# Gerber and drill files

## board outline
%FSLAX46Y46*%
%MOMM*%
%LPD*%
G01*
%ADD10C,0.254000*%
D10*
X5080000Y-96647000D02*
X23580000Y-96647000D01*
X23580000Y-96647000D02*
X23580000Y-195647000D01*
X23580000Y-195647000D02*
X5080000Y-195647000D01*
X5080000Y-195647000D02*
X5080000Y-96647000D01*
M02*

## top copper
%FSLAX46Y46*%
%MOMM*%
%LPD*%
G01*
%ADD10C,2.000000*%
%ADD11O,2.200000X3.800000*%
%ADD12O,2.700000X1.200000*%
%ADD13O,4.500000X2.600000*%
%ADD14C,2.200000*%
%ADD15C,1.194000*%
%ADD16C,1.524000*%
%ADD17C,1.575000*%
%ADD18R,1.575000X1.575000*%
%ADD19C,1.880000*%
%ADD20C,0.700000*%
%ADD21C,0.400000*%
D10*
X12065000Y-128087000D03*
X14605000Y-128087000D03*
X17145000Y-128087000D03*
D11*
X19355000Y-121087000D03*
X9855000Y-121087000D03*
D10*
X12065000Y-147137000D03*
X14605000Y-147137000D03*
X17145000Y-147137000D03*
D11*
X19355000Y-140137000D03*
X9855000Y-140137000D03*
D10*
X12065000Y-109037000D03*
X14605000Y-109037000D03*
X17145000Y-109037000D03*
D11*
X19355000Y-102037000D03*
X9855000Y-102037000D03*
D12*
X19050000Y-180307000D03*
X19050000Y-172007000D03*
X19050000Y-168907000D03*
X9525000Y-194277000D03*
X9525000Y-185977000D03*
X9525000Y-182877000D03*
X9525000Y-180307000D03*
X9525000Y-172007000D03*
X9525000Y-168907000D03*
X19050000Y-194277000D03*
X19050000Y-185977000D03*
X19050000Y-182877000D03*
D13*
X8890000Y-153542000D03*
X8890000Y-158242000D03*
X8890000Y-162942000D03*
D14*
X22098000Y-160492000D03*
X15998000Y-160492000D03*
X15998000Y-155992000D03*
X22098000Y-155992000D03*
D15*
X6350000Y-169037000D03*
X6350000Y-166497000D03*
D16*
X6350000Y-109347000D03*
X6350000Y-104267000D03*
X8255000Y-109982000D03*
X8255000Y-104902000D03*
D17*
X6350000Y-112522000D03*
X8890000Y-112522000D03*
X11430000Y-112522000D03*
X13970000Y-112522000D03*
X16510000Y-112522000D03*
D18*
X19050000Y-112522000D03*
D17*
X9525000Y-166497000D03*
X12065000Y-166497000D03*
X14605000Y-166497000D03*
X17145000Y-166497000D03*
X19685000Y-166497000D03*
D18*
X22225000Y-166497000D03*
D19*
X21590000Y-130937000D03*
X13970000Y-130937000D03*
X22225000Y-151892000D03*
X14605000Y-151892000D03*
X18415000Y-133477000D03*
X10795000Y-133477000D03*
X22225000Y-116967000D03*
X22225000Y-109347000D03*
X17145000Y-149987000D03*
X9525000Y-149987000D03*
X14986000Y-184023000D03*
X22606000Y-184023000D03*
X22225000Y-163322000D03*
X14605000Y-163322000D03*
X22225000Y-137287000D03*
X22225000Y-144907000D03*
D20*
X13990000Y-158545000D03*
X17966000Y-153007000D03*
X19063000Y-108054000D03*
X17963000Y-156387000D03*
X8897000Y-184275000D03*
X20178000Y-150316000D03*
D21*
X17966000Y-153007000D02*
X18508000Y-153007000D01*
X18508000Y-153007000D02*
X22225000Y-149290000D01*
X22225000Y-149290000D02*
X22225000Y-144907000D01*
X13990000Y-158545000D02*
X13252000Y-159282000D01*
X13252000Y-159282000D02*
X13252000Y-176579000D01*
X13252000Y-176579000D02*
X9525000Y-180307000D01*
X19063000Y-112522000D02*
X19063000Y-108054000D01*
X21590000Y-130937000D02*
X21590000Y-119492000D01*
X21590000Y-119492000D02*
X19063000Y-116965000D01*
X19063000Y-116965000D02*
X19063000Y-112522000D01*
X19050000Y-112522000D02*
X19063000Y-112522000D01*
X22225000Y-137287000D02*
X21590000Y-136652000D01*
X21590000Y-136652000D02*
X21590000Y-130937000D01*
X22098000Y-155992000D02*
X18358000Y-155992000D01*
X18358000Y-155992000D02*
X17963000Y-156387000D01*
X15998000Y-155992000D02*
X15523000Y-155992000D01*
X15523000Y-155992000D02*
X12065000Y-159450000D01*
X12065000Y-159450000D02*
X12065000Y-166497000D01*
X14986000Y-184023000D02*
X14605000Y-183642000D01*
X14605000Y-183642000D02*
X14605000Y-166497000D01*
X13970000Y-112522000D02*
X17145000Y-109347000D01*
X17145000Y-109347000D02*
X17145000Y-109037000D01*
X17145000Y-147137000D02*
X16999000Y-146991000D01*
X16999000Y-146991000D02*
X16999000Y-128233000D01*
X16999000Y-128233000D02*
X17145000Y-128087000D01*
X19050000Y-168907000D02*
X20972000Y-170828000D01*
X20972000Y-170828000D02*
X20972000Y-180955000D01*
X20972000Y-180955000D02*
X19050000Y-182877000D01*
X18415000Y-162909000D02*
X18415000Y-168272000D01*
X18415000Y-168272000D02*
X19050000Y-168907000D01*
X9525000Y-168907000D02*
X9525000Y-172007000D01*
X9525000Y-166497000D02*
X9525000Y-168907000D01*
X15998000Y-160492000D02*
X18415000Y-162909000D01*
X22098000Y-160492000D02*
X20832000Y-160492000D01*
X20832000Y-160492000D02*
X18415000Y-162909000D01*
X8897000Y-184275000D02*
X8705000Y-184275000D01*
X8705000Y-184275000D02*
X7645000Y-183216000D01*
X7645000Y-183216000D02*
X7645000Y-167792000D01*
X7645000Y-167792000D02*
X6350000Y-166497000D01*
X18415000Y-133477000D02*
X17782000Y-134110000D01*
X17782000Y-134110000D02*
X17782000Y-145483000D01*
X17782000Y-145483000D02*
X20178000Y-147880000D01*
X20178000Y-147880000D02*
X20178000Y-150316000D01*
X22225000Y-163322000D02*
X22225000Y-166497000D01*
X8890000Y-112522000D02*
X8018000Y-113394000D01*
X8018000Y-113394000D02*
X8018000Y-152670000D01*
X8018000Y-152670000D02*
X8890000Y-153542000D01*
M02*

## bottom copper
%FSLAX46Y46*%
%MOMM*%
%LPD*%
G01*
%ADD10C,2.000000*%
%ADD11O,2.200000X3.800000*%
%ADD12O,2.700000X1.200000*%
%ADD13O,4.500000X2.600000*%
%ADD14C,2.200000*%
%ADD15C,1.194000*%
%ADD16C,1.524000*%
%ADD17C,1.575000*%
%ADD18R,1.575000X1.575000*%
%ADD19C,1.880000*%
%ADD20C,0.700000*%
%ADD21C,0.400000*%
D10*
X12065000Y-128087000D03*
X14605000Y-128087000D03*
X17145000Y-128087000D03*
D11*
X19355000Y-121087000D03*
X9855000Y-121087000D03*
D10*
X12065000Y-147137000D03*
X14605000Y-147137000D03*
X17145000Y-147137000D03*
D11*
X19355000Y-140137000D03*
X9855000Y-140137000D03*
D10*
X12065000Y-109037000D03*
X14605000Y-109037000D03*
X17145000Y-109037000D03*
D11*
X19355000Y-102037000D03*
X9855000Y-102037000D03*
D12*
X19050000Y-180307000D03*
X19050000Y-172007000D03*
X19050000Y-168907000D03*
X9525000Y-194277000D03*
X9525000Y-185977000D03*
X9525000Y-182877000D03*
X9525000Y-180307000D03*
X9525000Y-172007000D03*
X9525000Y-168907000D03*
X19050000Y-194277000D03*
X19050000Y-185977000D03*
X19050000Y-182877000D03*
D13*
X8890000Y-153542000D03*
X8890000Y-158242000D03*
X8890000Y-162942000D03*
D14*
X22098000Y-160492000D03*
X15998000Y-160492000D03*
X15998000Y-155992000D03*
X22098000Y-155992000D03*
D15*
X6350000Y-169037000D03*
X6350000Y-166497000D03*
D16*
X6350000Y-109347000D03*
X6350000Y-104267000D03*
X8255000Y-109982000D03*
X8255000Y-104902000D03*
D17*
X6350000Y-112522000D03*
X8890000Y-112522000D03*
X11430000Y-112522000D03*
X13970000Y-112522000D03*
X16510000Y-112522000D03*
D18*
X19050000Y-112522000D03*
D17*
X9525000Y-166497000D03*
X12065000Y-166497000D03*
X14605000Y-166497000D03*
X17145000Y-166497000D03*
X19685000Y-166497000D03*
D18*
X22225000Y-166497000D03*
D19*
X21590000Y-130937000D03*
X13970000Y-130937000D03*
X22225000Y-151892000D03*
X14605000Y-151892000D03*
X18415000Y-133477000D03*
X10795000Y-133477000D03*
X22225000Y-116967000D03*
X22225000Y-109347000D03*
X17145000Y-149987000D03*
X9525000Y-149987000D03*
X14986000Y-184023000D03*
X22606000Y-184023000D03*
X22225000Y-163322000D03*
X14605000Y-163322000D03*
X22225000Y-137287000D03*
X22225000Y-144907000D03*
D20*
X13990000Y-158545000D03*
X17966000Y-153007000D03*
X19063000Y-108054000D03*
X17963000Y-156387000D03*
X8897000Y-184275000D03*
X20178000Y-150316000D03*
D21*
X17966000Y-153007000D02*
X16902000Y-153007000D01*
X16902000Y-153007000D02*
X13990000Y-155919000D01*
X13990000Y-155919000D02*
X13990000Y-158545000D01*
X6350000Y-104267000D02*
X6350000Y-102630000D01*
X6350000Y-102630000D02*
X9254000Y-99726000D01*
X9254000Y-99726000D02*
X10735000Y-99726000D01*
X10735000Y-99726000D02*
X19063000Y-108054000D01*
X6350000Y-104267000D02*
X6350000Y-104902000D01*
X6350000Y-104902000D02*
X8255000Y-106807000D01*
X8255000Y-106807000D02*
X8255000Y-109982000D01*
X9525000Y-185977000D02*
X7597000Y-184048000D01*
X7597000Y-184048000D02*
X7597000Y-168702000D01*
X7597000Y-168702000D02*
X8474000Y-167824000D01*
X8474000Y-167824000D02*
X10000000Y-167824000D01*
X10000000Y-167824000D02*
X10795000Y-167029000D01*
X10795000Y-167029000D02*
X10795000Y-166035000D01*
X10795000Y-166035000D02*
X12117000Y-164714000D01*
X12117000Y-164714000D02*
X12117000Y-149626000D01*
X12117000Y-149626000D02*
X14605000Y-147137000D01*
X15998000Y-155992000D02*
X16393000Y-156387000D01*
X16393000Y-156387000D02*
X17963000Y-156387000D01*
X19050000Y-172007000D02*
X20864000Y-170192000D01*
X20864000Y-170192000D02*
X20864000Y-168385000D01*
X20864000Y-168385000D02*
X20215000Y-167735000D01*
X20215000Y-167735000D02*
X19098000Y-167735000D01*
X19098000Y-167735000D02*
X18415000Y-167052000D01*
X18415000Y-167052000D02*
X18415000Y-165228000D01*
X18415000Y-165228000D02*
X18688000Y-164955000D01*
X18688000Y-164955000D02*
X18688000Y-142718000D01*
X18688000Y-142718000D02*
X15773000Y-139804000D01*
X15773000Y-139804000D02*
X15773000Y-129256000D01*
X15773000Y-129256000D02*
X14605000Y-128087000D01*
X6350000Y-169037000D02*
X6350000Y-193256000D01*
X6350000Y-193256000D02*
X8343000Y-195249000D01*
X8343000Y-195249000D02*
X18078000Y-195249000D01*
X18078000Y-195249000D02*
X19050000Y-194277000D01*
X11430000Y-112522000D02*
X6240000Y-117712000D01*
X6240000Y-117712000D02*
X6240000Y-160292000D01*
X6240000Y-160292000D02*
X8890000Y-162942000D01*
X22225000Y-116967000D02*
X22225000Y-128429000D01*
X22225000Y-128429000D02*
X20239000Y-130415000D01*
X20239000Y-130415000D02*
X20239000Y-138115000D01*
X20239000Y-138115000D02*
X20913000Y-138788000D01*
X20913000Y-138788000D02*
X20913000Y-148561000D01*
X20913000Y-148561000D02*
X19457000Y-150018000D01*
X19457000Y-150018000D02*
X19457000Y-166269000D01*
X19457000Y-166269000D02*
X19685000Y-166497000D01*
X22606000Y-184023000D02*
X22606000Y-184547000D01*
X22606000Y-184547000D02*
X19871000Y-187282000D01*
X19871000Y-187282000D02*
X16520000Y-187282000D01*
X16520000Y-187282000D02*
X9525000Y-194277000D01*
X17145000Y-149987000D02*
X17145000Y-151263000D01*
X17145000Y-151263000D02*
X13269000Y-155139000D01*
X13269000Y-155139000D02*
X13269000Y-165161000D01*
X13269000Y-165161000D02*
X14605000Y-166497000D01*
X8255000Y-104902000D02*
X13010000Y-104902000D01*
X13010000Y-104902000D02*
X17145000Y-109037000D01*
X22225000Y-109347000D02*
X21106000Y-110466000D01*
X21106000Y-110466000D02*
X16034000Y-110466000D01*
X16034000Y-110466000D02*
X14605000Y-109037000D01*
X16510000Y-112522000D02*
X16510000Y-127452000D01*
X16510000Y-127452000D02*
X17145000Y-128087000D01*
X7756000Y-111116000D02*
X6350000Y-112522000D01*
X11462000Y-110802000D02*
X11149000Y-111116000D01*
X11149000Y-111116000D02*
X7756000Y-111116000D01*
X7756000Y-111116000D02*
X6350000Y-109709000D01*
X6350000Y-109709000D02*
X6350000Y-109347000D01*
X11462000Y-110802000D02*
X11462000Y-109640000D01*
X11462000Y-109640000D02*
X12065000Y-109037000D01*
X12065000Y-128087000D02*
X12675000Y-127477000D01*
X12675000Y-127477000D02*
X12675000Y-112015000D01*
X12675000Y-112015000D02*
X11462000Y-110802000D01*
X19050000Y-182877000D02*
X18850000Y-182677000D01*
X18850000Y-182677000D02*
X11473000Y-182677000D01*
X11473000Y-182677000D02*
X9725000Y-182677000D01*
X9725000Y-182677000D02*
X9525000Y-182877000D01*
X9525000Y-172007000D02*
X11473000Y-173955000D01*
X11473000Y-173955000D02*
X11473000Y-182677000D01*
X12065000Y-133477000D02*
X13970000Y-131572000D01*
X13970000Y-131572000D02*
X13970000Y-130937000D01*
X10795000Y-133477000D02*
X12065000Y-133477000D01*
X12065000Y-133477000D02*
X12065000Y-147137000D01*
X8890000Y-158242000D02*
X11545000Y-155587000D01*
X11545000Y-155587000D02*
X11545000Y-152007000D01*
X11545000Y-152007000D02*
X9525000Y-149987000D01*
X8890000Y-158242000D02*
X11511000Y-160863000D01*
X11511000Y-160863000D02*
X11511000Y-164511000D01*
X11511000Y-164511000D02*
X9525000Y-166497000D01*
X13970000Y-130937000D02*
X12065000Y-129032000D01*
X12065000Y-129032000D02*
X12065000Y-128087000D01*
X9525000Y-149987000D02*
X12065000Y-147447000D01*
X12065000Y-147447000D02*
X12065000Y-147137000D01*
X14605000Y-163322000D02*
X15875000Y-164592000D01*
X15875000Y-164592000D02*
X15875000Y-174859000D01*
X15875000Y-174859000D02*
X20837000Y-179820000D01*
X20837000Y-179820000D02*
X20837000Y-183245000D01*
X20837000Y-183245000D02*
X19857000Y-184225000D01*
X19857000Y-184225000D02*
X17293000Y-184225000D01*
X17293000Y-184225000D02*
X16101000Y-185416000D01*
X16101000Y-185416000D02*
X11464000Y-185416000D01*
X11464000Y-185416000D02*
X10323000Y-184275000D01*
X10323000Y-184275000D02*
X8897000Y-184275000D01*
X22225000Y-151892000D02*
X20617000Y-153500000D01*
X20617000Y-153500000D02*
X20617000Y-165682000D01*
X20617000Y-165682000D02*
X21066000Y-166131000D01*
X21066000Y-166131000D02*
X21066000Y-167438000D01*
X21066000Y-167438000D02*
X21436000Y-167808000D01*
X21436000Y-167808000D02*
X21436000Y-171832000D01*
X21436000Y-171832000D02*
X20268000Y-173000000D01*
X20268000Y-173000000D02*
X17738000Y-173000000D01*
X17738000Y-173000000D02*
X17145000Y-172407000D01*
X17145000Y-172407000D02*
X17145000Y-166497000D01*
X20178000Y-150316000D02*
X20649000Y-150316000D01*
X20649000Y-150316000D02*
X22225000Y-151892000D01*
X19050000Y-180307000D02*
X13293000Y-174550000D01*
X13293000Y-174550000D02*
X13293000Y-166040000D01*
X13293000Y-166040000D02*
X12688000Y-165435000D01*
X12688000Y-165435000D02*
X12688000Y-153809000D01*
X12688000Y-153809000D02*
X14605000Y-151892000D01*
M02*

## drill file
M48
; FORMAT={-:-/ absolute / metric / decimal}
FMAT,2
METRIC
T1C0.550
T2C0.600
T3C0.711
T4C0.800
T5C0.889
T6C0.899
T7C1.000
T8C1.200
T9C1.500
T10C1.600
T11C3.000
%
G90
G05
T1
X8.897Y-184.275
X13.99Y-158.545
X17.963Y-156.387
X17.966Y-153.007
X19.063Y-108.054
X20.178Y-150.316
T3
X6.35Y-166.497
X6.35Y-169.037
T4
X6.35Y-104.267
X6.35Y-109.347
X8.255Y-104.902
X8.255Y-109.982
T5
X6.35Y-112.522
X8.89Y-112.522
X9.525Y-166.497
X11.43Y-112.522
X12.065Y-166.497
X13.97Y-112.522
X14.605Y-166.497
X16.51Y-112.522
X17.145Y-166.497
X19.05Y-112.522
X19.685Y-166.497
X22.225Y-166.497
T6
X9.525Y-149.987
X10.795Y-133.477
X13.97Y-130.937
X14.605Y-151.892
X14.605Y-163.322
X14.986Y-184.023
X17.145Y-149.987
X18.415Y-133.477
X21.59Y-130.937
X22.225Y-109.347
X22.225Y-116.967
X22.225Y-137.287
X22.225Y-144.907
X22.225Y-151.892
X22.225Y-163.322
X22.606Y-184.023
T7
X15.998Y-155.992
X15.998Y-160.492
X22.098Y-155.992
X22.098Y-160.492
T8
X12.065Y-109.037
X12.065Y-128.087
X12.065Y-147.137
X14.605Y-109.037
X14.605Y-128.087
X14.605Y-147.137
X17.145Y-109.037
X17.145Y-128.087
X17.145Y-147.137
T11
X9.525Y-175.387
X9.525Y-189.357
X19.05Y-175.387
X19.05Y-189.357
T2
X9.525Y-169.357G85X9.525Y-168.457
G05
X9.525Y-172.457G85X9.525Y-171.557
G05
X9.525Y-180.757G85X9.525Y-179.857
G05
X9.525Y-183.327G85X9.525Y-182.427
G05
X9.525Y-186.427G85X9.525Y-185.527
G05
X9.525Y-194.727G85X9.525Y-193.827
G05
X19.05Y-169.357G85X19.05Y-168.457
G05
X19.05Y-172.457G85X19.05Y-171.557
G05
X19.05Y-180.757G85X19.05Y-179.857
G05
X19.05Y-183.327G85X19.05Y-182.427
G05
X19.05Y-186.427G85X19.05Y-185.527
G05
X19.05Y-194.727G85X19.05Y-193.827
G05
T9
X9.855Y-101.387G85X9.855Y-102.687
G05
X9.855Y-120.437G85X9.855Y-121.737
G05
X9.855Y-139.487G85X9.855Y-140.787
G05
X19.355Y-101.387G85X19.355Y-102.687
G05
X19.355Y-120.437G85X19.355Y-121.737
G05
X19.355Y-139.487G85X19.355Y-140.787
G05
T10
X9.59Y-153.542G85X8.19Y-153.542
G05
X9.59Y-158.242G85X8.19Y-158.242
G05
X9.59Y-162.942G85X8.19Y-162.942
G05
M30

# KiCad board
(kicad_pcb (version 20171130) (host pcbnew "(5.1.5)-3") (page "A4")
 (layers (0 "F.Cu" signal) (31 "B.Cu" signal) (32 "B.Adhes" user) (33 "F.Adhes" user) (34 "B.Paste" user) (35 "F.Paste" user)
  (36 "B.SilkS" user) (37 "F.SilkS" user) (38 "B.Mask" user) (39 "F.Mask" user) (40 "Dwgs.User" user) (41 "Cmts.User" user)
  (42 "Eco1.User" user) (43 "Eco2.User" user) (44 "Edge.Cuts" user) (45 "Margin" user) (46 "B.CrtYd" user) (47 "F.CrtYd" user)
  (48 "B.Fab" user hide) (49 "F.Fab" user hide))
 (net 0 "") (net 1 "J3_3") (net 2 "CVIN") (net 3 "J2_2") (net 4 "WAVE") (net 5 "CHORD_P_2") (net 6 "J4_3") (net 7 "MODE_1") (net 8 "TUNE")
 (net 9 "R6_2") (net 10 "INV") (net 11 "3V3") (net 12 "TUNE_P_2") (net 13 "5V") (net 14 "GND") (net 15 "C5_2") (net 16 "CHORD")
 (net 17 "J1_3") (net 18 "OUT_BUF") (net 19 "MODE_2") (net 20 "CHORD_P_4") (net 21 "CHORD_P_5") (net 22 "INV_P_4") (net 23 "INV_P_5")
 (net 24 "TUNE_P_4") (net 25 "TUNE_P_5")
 (segment (start 17.966 153.007) (end 16.902 153.007) (width 0.4) (layer "B.Cu") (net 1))
 (segment (start 16.902 153.007) (end 13.99 155.919) (width 0.4) (layer "B.Cu") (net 1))
 (segment (start 13.99 155.919) (end 13.99 158.545) (width 0.4) (layer "B.Cu") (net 1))
 (segment (start 6.35 104.267) (end 6.35 102.63) (width 0.4) (layer "B.Cu") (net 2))
 (segment (start 6.35 102.63) (end 9.254 99.726) (width 0.4) (layer "B.Cu") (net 2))
 (segment (start 9.254 99.726) (end 10.735 99.726) (width 0.4) (layer "B.Cu") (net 2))
 (segment (start 10.735 99.726) (end 19.063 108.054) (width 0.4) (layer "B.Cu") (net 2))
 (segment (start 6.35 104.267) (end 6.35 104.902) (width 0.4) (layer "B.Cu") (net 2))
 (segment (start 6.35 104.902) (end 8.255 106.807) (width 0.4) (layer "B.Cu") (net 2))
 (segment (start 8.255 106.807) (end 8.255 109.982) (width 0.4) (layer "B.Cu") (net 2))
 (segment (start 9.525 185.977) (end 7.597 184.048) (width 0.4) (layer "B.Cu") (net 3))
 (segment (start 7.597 184.048) (end 7.597 168.702) (width 0.4) (layer "B.Cu") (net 3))
 (segment (start 7.597 168.702) (end 8.474 167.824) (width 0.4) (layer "B.Cu") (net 3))
 (segment (start 8.474 167.824) (end 10 167.824) (width 0.4) (layer "B.Cu") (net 3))
 (segment (start 10 167.824) (end 10.795 167.029) (width 0.4) (layer "B.Cu") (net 3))
 (segment (start 10.795 167.029) (end 10.795 166.035) (width 0.4) (layer "B.Cu") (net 3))
 (segment (start 10.795 166.035) (end 12.117 164.714) (width 0.4) (layer "B.Cu") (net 3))
 (segment (start 12.117 164.714) (end 12.117 149.626) (width 0.4) (layer "B.Cu") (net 3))
 (segment (start 12.117 149.626) (end 14.605 147.137) (width 0.4) (layer "B.Cu") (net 3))
 (segment (start 15.998 155.992) (end 16.393 156.387) (width 0.4) (layer "B.Cu") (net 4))
 (segment (start 16.393 156.387) (end 17.963 156.387) (width 0.4) (layer "B.Cu") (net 4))
 (segment (start 19.05 172.007) (end 20.864 170.192) (width 0.4) (layer "B.Cu") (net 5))
 (segment (start 20.864 170.192) (end 20.864 168.385) (width 0.4) (layer "B.Cu") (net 5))
 (segment (start 20.864 168.385) (end 20.215 167.735) (width 0.4) (layer "B.Cu") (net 5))
 (segment (start 20.215 167.735) (end 19.098 167.735) (width 0.4) (layer "B.Cu") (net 5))
 (segment (start 19.098 167.735) (end 18.415 167.052) (width 0.4) (layer "B.Cu") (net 5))
 (segment (start 18.415 167.052) (end 18.415 165.228) (width 0.4) (layer "B.Cu") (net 5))
 (segment (start 18.415 165.228) (end 18.688 164.955) (width 0.4) (layer "B.Cu") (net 5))
 (segment (start 18.688 164.955) (end 18.688 142.718) (width 0.4) (layer "B.Cu") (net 5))
 (segment (start 18.688 142.718) (end 15.773 139.804) (width 0.4) (layer "B.Cu") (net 5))
 (segment (start 15.773 139.804) (end 15.773 129.256) (width 0.4) (layer "B.Cu") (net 5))
 (segment (start 15.773 129.256) (end 14.605 128.087) (width 0.4) (layer "B.Cu") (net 5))
 (segment (start 6.35 169.037) (end 6.35 193.256) (width 0.4) (layer "B.Cu") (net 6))
 (segment (start 6.35 193.256) (end 8.343 195.249) (width 0.4) (layer "B.Cu") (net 6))
 (segment (start 8.343 195.249) (end 18.078 195.249) (width 0.4) (layer "B.Cu") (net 6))
 (segment (start 18.078 195.249) (end 19.05 194.277) (width 0.4) (layer "B.Cu") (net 6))
 (segment (start 11.43 112.522) (end 6.24 117.712) (width 0.4) (layer "B.Cu") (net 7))
 (segment (start 6.24 117.712) (end 6.24 160.292) (width 0.4) (layer "B.Cu") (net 7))
 (segment (start 6.24 160.292) (end 8.89 162.942) (width 0.4) (layer "B.Cu") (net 7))
 (segment (start 22.225 116.967) (end 22.225 128.429) (width 0.4) (layer "B.Cu") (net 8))
 (segment (start 22.225 128.429) (end 20.239 130.415) (width 0.4) (layer "B.Cu") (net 8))
 (segment (start 20.239 130.415) (end 20.239 138.115) (width 0.4) (layer "B.Cu") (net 8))
 (segment (start 20.239 138.115) (end 20.913 138.788) (width 0.4) (layer "B.Cu") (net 8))
 (segment (start 20.913 138.788) (end 20.913 148.561) (width 0.4) (layer "B.Cu") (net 8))
 (segment (start 20.913 148.561) (end 19.457 150.018) (width 0.4) (layer "B.Cu") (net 8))
 (segment (start 19.457 150.018) (end 19.457 166.269) (width 0.4) (layer "B.Cu") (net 8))
 (segment (start 19.457 166.269) (end 19.685 166.497) (width 0.4) (layer "B.Cu") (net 8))
 (segment (start 22.606 184.023) (end 22.606 184.547) (width 0.4) (layer "B.Cu") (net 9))
 (segment (start 22.606 184.547) (end 19.871 187.282) (width 0.4) (layer "B.Cu") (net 9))
 (segment (start 19.871 187.282) (end 16.52 187.282) (width 0.4) (layer "B.Cu") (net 9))
 (segment (start 16.52 187.282) (end 9.525 194.277) (width 0.4) (layer "B.Cu") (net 9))
 (segment (start 17.145 149.987) (end 17.145 151.263) (width 0.4) (layer "B.Cu") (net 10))
 (segment (start 17.145 151.263) (end 13.269 155.139) (width 0.4) (layer "B.Cu") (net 10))
 (segment (start 13.269 155.139) (end 13.269 165.161) (width 0.4) (layer "B.Cu") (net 10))
 (segment (start 13.269 165.161) (end 14.605 166.497) (width 0.4) (layer "B.Cu") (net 10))
 (segment (start 8.255 104.902) (end 13.01 104.902) (width 0.4) (layer "B.Cu") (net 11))
 (segment (start 13.01 104.902) (end 17.145 109.037) (width 0.4) (layer "B.Cu") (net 11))
 (segment (start 22.225 109.347) (end 21.106 110.466) (width 0.4) (layer "B.Cu") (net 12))
 (segment (start 21.106 110.466) (end 16.034 110.466) (width 0.4) (layer "B.Cu") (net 12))
 (segment (start 16.034 110.466) (end 14.605 109.037) (width 0.4) (layer "B.Cu") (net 12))
 (segment (start 16.51 112.522) (end 16.51 127.452) (width 0.4) (layer "B.Cu") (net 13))
 (segment (start 16.51 127.452) (end 17.145 128.087) (width 0.4) (layer "B.Cu") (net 13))
 (segment (start 7.756 111.116) (end 6.35 112.522) (width 0.4) (layer "B.Cu") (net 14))
 (segment (start 11.462 110.802) (end 11.149 111.116) (width 0.4) (layer "B.Cu") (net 14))
 (segment (start 11.149 111.116) (end 7.756 111.116) (width 0.4) (layer "B.Cu") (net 14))
 (segment (start 7.756 111.116) (end 6.35 109.709) (width 0.4) (layer "B.Cu") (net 14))
 (segment (start 6.35 109.709) (end 6.35 109.347) (width 0.4) (layer "B.Cu") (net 14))
 (segment (start 11.462 110.802) (end 11.462 109.64) (width 0.4) (layer "B.Cu") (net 14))
 (segment (start 11.462 109.64) (end 12.065 109.037) (width 0.4) (layer "B.Cu") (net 14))
 (segment (start 12.065 128.087) (end 12.675 127.477) (width 0.4) (layer "B.Cu") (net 14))
 (segment (start 12.675 127.477) (end 12.675 112.015) (width 0.4) (layer "B.Cu") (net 14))
 (segment (start 12.675 112.015) (end 11.462 110.802) (width 0.4) (layer "B.Cu") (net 14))
 (segment (start 19.05 182.877) (end 18.85 182.677) (width 0.4) (layer "B.Cu") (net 14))
 (segment (start 18.85 182.677) (end 11.473 182.677) (width 0.4) (layer "B.Cu") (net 14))
 (segment (start 11.473 182.677) (end 9.725 182.677) (width 0.4) (layer "B.Cu") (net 14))
 (segment (start 9.725 182.677) (end 9.525 182.877) (width 0.4) (layer "B.Cu") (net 14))
 (segment (start 9.525 172.007) (end 11.473 173.955) (width 0.4) (layer "B.Cu") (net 14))
 (segment (start 11.473 173.955) (end 11.473 182.677) (width 0.4) (layer "B.Cu") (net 14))
 (segment (start 12.065 133.477) (end 13.97 131.572) (width 0.4) (layer "B.Cu") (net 14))
 (segment (start 13.97 131.572) (end 13.97 130.937) (width 0.4) (layer "B.Cu") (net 14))
 (segment (start 10.795 133.477) (end 12.065 133.477) (width 0.4) (layer "B.Cu") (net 14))
 (segment (start 12.065 133.477) (end 12.065 147.137) (width 0.4) (layer "B.Cu") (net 14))
 (segment (start 8.89 158.242) (end 11.545 155.587) (width 0.4) (layer "B.Cu") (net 14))
 (segment (start 11.545 155.587) (end 11.545 152.007) (width 0.4) (layer "B.Cu") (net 14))
 (segment (start 11.545 152.007) (end 9.525 149.987) (width 0.4) (layer "B.Cu") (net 14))
 (segment (start 8.89 158.242) (end 11.511 160.863) (width 0.4) (layer "B.Cu") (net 14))
 (segment (start 11.511 160.863) (end 11.511 164.511) (width 0.4) (layer "B.Cu") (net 14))
 (segment (start 11.511 164.511) (end 9.525 166.497) (width 0.4) (layer "B.Cu") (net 14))
 (segment (start 13.97 130.937) (end 12.065 129.032) (width 0.4) (layer "B.Cu") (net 14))
 (segment (start 12.065 129.032) (end 12.065 128.087) (width 0.4) (layer "B.Cu") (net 14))
 (segment (start 9.525 149.987) (end 12.065 147.447) (width 0.4) (layer "B.Cu") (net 14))
 (segment (start 12.065 147.447) (end 12.065 147.137) (width 0.4) (layer "B.Cu") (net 14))
 (segment (start 14.605 163.322) (end 15.875 164.592) (width 0.4) (layer "B.Cu") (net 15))
 (segment (start 15.875 164.592) (end 15.875 174.859) (width 0.4) (layer "B.Cu") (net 15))
 (segment (start 15.875 174.859) (end 20.837 179.82) (width 0.4) (layer "B.Cu") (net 15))
 (segment (start 20.837 179.82) (end 20.837 183.245) (width 0.4) (layer "B.Cu") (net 15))
 (segment (start 20.837 183.245) (end 19.857 184.225) (width 0.4) (layer "B.Cu") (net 15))
 (segment (start 19.857 184.225) (end 17.293 184.225) (width 0.4) (layer "B.Cu") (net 15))
 (segment (start 17.293 184.225) (end 16.101 185.416) (width 0.4) (layer "B.Cu") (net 15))
 (segment (start 16.101 185.416) (end 11.464 185.416) (width 0.4) (layer "B.Cu") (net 15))
 (segment (start 11.464 185.416) (end 10.323 184.275) (width 0.4) (layer "B.Cu") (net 15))
 (segment (start 10.323 184.275) (end 8.897 184.275) (width 0.4) (layer "B.Cu") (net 15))
 (segment (start 22.225 151.892) (end 20.617 153.5) (width 0.4) (layer "B.Cu") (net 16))
 (segment (start 20.617 153.5) (end 20.617 165.682) (width 0.4) (layer "B.Cu") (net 16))
 (segment (start 20.617 165.682) (end 21.066 166.131) (width 0.4) (layer "B.Cu") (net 16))
 (segment (start 21.066 166.131) (end 21.066 167.438) (width 0.4) (layer "B.Cu") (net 16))
 (segment (start 21.066 167.438) (end 21.436 167.808) (width 0.4) (layer "B.Cu") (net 16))
 (segment (start 21.436 167.808) (end 21.436 171.832) (width 0.4) (layer "B.Cu") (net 16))
 (segment (start 21.436 171.832) (end 20.268 173) (width 0.4) (layer "B.Cu") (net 16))
 (segment (start 20.268 173) (end 17.738 173) (width 0.4) (layer "B.Cu") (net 16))
 (segment (start 17.738 173) (end 17.145 172.407) (width 0.4) (layer "B.Cu") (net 16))
 (segment (start 17.145 172.407) (end 17.145 166.497) (width 0.4) (layer "B.Cu") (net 16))
 (segment (start 20.178 150.316) (end 20.649 150.316) (width 0.4) (layer "B.Cu") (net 16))
 (segment (start 20.649 150.316) (end 22.225 151.892) (width 0.4) (layer "B.Cu") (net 16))
 (segment (start 19.05 180.307) (end 13.293 174.55) (width 0.4) (layer "B.Cu") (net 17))
 (segment (start 13.293 174.55) (end 13.293 166.04) (width 0.4) (layer "B.Cu") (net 17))
 (segment (start 13.293 166.04) (end 12.688 165.435) (width 0.4) (layer "B.Cu") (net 17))
 (segment (start 12.688 165.435) (end 12.688 153.809) (width 0.4) (layer "B.Cu") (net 17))
 (segment (start 12.688 153.809) (end 14.605 151.892) (width 0.4) (layer "B.Cu") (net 17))
 (gr_line (start 5.08 96.647) (end 23.58 96.647) (width 0.254) (layer "Edge.Cuts"))
 (gr_line (start 23.58 96.647) (end 23.58 195.647) (width 0.254) (layer "Edge.Cuts"))
 (gr_line (start 23.58 195.647) (end 5.08 195.647) (width 0.254) (layer "Edge.Cuts"))
 (gr_line (start 5.08 195.647) (end 5.08 96.647) (width 0.254) (layer "Edge.Cuts"))
 (segment (start 17.966 153.007) (end 18.508 153.007) (width 0.4) (layer "F.Cu") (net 1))
 (segment (start 18.508 153.007) (end 22.225 149.29) (width 0.4) (layer "F.Cu") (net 1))
 (segment (start 22.225 149.29) (end 22.225 144.907) (width 0.4) (layer "F.Cu") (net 1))
 (segment (start 13.99 158.545) (end 13.252 159.282) (width 0.4) (layer "F.Cu") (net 1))
 (segment (start 13.252 159.282) (end 13.252 176.579) (width 0.4) (layer "F.Cu") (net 1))
 (segment (start 13.252 176.579) (end 9.525 180.307) (width 0.4) (layer "F.Cu") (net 1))
 (segment (start 19.063 112.522) (end 19.063 108.054) (width 0.4) (layer "F.Cu") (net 2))
 (segment (start 21.59 130.937) (end 21.59 119.492) (width 0.4) (layer "F.Cu") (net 2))
 (segment (start 21.59 119.492) (end 19.063 116.965) (width 0.4) (layer "F.Cu") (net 2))
 (segment (start 19.063 116.965) (end 19.063 112.522) (width 0.4) (layer "F.Cu") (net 2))
 (segment (start 19.05 112.522) (end 19.063 112.522) (width 0.4) (layer "F.Cu") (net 2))
 (segment (start 22.225 137.287) (end 21.59 136.652) (width 0.4) (layer "F.Cu") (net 2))
 (segment (start 21.59 136.652) (end 21.59 130.937) (width 0.4) (layer "F.Cu") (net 2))
 (segment (start 22.098 155.992) (end 18.358 155.992) (width 0.4) (layer "F.Cu") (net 4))
 (segment (start 18.358 155.992) (end 17.963 156.387) (width 0.4) (layer "F.Cu") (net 4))
 (segment (start 15.998 155.992) (end 15.523 155.992) (width 0.4) (layer "F.Cu") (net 4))
 (segment (start 15.523 155.992) (end 12.065 159.45) (width 0.4) (layer "F.Cu") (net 4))
 (segment (start 12.065 159.45) (end 12.065 166.497) (width 0.4) (layer "F.Cu") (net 4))
 (segment (start 14.986 184.023) (end 14.605 183.642) (width 0.4) (layer "F.Cu") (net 10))
 (segment (start 14.605 183.642) (end 14.605 166.497) (width 0.4) (layer "F.Cu") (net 10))
 (segment (start 13.97 112.522) (end 17.145 109.347) (width 0.4) (layer "F.Cu") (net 11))
 (segment (start 17.145 109.347) (end 17.145 109.037) (width 0.4) (layer "F.Cu") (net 11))
 (segment (start 17.145 147.137) (end 16.999 146.991) (width 0.4) (layer "F.Cu") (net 13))
 (segment (start 16.999 146.991) (end 16.999 128.233) (width 0.4) (layer "F.Cu") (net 13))
 (segment (start 16.999 128.233) (end 17.145 128.087) (width 0.4) (layer "F.Cu") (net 13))
 (segment (start 19.05 168.907) (end 20.972 170.828) (width 0.4) (layer "F.Cu") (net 14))
 (segment (start 20.972 170.828) (end 20.972 180.955) (width 0.4) (layer "F.Cu") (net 14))
 (segment (start 20.972 180.955) (end 19.05 182.877) (width 0.4) (layer "F.Cu") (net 14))
 (segment (start 18.415 162.909) (end 18.415 168.272) (width 0.4) (layer "F.Cu") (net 14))
 (segment (start 18.415 168.272) (end 19.05 168.907) (width 0.4) (layer "F.Cu") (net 14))
 (segment (start 9.525 168.907) (end 9.525 172.007) (width 0.4) (layer "F.Cu") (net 14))
 (segment (start 9.525 166.497) (end 9.525 168.907) (width 0.4) (layer "F.Cu") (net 14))
 (segment (start 15.998 160.492) (end 18.415 162.909) (width 0.4) (layer "F.Cu") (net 14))
 (segment (start 22.098 160.492) (end 20.832 160.492) (width 0.4) (layer "F.Cu") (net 14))
 (segment (start 20.832 160.492) (end 18.415 162.909) (width 0.4) (layer "F.Cu") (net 14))
 (segment (start 8.897 184.275) (end 8.705 184.275) (width 0.4) (layer "F.Cu") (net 15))
 (segment (start 8.705 184.275) (end 7.645 183.216) (width 0.4) (layer "F.Cu") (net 15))
 (segment (start 7.645 183.216) (end 7.645 167.792) (width 0.4) (layer "F.Cu") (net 15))
 (segment (start 7.645 167.792) (end 6.35 166.497) (width 0.4) (layer "F.Cu") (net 15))
 (segment (start 18.415 133.477) (end 17.782 134.11) (width 0.4) (layer "F.Cu") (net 16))
 (segment (start 17.782 134.11) (end 17.782 145.483) (width 0.4) (layer "F.Cu") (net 16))
 (segment (start 17.782 145.483) (end 20.178 147.88) (width 0.4) (layer "F.Cu") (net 16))
 (segment (start 20.178 147.88) (end 20.178 150.316) (width 0.4) (layer "F.Cu") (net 16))
 (segment (start 22.225 163.322) (end 22.225 166.497) (width 0.4) (layer "F.Cu") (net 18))
 (segment (start 8.89 112.522) (end 8.018 113.394) (width 0.4) (layer "F.Cu") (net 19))
 (segment (start 8.018 113.394) (end 8.018 152.67) (width 0.4) (layer "F.Cu") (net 19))
 (segment (start 8.018 152.67) (end 8.89 153.542) (width 0.4) (layer "F.Cu") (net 19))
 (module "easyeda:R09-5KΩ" (layer "F.Cu") (at 14.605 124.587)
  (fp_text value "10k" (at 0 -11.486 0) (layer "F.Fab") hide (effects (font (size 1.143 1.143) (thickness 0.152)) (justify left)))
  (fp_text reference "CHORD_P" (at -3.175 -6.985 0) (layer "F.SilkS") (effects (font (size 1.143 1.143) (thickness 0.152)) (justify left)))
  (pad 1 thru_hole circle (at -2.54 3.5 0) (size 2 2) (layers "*.Cu" "*.Paste" "*.Mask") (drill 1.2) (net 14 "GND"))
  (pad 2 thru_hole circle (at 0 3.5 0) (size 2 2) (layers "*.Cu" "*.Paste" "*.Mask") (drill 1.2) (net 5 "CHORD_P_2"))
  (pad 3 thru_hole circle (at 2.54 3.5 0) (size 2 2) (layers "*.Cu" "*.Paste" "*.Mask") (drill 1.2) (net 13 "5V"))
  (pad 4 thru_hole oval (at 4.75 -3.5 0) (size 2.2 3.8) (layers "*.Cu" "*.Paste" "*.Mask") (drill oval 1.5 2.8) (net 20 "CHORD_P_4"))
  (pad 5 thru_hole oval (at -4.75 -3.5 0) (size 2.2 3.8) (layers "*.Cu" "*.Paste" "*.Mask") (drill oval 1.5 2.8) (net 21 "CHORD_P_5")))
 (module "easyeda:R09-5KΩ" (layer "F.Cu") (at 14.605 143.637)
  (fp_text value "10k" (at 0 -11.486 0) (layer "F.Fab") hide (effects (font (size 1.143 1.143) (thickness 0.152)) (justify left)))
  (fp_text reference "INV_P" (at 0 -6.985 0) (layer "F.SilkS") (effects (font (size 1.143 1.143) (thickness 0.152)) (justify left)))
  (pad 1 thru_hole circle (at -2.54 3.5 0) (size 2 2) (layers "*.Cu" "*.Paste" "*.Mask") (drill 1.2) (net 14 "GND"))
  (pad 2 thru_hole circle (at 0 3.5 0) (size 2 2) (layers "*.Cu" "*.Paste" "*.Mask") (drill 1.2) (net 3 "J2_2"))
  (pad 3 thru_hole circle (at 2.54 3.5 0) (size 2 2) (layers "*.Cu" "*.Paste" "*.Mask") (drill 1.2) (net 13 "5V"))
  (pad 4 thru_hole oval (at 4.75 -3.5 0) (size 2.2 3.8) (layers "*.Cu" "*.Paste" "*.Mask") (drill oval 1.5 2.8) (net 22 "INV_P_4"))
  (pad 5 thru_hole oval (at -4.75 -3.5 0) (size 2.2 3.8) (layers "*.Cu" "*.Paste" "*.Mask") (drill oval 1.5 2.8) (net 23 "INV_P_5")))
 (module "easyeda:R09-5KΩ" (layer "F.Cu") (at 14.605 105.537)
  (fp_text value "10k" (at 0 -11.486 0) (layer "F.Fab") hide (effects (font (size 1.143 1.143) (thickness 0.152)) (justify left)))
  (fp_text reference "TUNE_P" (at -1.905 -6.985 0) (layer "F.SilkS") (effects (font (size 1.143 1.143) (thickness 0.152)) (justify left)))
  (pad 1 thru_hole circle (at -2.54 3.5 0) (size 2 2) (layers "*.Cu" "*.Paste" "*.Mask") (drill 1.2) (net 14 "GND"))
  (pad 2 thru_hole circle (at 0 3.5 0) (size 2 2) (layers "*.Cu" "*.Paste" "*.Mask") (drill 1.2) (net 12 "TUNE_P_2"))
  (pad 3 thru_hole circle (at 2.54 3.5 0) (size 2 2) (layers "*.Cu" "*.Paste" "*.Mask") (drill 1.2) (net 11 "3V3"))
  (pad 4 thru_hole oval (at 4.75 -3.5 0) (size 2.2 3.8) (layers "*.Cu" "*.Paste" "*.Mask") (drill oval 1.5 2.8) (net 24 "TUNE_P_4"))
  (pad 5 thru_hole oval (at -4.75 -3.5 0) (size 2.2 3.8) (layers "*.Cu" "*.Paste" "*.Mask") (drill oval 1.5 2.8) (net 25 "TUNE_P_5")))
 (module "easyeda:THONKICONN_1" (layer "F.Cu") (at 19.05 175.387 180)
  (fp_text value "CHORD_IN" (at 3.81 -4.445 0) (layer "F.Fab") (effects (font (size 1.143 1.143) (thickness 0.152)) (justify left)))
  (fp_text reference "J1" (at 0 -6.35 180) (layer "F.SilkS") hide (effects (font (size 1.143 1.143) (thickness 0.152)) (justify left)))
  (pad "" np_thru_hole circle (at 0 0) (size 3 3) (drill 3) (layers "*.Cu" "*.Mask"))
  (pad 3 thru_hole oval (at 0 -4.92 180) (size 2.7 1.2) (layers "*.Cu" "*.Paste" "*.Mask") (drill oval 0.6 1.5) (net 17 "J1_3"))
  (pad 2 thru_hole oval (at 0 3.38 180) (size 2.7 1.2) (layers "*.Cu" "*.Paste" "*.Mask") (drill oval 0.6 1.5) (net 5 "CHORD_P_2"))
  (pad 1 thru_hole oval (at 0 6.48 180) (size 2.7 1.2) (layers "*.Cu" "*.Paste" "*.Mask") (drill oval 0.6 1.5) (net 14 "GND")))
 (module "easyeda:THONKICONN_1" (layer "F.Cu") (at 9.525 189.357 180)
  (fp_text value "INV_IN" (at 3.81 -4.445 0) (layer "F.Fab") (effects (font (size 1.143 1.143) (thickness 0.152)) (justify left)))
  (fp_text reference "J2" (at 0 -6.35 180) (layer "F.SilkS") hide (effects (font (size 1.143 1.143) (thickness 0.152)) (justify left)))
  (pad "" np_thru_hole circle (at 0 0) (size 3 3) (drill 3) (layers "*.Cu" "*.Mask"))
  (pad 3 thru_hole oval (at 0 -4.92 180) (size 2.7 1.2) (layers "*.Cu" "*.Paste" "*.Mask") (drill oval 0.6 1.5) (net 9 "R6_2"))
  (pad 2 thru_hole oval (at 0 3.38 180) (size 2.7 1.2) (layers "*.Cu" "*.Paste" "*.Mask") (drill oval 0.6 1.5) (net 3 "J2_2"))
  (pad 1 thru_hole oval (at 0 6.48 180) (size 2.7 1.2) (layers "*.Cu" "*.Paste" "*.Mask") (drill oval 0.6 1.5) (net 14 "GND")))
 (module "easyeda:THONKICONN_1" (layer "F.Cu") (at 9.525 175.387 180)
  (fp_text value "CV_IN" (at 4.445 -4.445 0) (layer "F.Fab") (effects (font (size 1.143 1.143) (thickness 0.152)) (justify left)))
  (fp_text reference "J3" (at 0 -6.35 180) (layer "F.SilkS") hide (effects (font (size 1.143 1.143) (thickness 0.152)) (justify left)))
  (pad "" np_thru_hole circle (at 0 0) (size 3 3) (drill 3) (layers "*.Cu" "*.Mask"))
  (pad 3 thru_hole oval (at 0 -4.92 180) (size 2.7 1.2) (layers "*.Cu" "*.Paste" "*.Mask") (drill oval 0.6 1.5) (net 1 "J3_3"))
  (pad 2 thru_hole oval (at 0 3.38 180) (size 2.7 1.2) (layers "*.Cu" "*.Paste" "*.Mask") (drill oval 0.6 1.5) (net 14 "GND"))
  (pad 1 thru_hole oval (at 0 6.48 180) (size 2.7 1.2) (layers "*.Cu" "*.Paste" "*.Mask") (drill oval 0.6 1.5) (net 14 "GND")))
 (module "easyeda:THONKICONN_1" (layer "F.Cu") (at 19.05 189.357 180)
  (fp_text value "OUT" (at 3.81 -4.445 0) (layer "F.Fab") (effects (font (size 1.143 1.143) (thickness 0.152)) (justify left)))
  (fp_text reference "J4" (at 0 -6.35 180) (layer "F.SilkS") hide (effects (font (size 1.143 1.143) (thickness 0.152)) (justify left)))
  (pad "" np_thru_hole circle (at 0 0) (size 3 3) (drill 3) (layers "*.Cu" "*.Mask"))
  (pad 3 thru_hole oval (at 0 -4.92 180) (size 2.7 1.2) (layers "*.Cu" "*.Paste" "*.Mask") (drill oval 0.6 1.5) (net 6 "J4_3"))
  (pad 2 thru_hole oval (at 0 3.38 180) (size 2.7 1.2) (layers "*.Cu" "*.Paste" "*.Mask") (drill oval 0.6 1.5))
  (pad 1 thru_hole oval (at 0 6.48 180) (size 2.7 1.2) (layers "*.Cu" "*.Paste" "*.Mask") (drill oval 0.6 1.5) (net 14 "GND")))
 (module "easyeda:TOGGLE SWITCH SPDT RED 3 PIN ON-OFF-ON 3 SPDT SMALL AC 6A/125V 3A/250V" (layer "F.Cu") (at 8.89 158.242)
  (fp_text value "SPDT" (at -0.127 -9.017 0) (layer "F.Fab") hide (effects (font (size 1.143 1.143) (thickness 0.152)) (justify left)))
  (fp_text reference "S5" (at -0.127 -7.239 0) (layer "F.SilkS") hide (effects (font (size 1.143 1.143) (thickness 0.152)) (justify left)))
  (pad 1 thru_hole oval (at 0 -4.7 -90) (size 2.6 4.5) (layers "*.Cu" "*.Paste" "*.Mask") (drill oval 1.6 3) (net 19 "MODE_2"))
  (pad 2 thru_hole oval (at 0 0 -90) (size 2.6 4.5) (layers "*.Cu" "*.Paste" "*.Mask") (drill oval 1.6 3) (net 14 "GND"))
  (pad 3 thru_hole oval (at 0 4.7 -90) (size 2.6 4.5) (layers "*.Cu" "*.Paste" "*.Mask") (drill oval 1.6 3) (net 7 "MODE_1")))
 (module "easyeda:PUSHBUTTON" (layer "F.Cu") (at 18.923 157.825)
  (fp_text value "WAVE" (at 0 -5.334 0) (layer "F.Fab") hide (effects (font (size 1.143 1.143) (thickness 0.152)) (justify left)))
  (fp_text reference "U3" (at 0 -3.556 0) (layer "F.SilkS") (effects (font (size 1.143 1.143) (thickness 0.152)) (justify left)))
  (pad 4 thru_hole circle (at 3.175 2.667 180) (size 2.2 2.2) (layers "*.Cu" "*.Paste" "*.Mask") (drill 1) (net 14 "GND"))
  (pad 3 thru_hole circle (at -2.925 2.667 180) (size 2.2 2.2) (layers "*.Cu" "*.Paste" "*.Mask") (drill 1) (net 14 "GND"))
  (pad 1 thru_hole circle (at -2.925 -1.833 180) (size 2.2 2.2) (layers "*.Cu" "*.Paste" "*.Mask") (drill 1) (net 4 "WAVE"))
  (pad 2 thru_hole circle (at 3.175 -1.833 180) (size 2.2 2.2) (layers "*.Cu" "*.Paste" "*.Mask") (drill 1) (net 4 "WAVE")))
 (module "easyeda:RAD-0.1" (layer "F.Cu") (at 6.35 167.767 -90)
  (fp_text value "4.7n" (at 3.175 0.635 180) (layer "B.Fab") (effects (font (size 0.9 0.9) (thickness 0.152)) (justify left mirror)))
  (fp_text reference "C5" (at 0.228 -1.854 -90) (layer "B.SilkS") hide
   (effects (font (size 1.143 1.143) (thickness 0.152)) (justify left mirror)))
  (pad 1 thru_hole circle (at 1.27 0 -90) (size 1.194 1.194) (layers "*.Cu" "*.Paste" "*.Mask") (drill 0.711) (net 6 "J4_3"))
  (pad 2 thru_hole circle (at -1.27 0 -90) (size 1.194 1.194) (layers "*.Cu" "*.Paste" "*.Mask") (drill 0.711) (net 15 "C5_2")))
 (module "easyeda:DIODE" (layer "F.Cu") (at 6.35 106.807 -90)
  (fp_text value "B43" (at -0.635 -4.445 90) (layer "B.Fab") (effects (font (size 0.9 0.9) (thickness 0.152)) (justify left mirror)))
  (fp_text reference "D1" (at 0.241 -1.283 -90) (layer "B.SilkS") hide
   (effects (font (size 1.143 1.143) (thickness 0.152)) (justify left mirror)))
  (pad 1 thru_hole circle (at 2.54 0 -90) (size 1.524 1.524) (layers "*.Cu" "*.Paste" "*.Mask") (drill 0.8) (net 14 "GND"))
  (pad 2 thru_hole circle (at -2.54 0 -90) (size 1.524 1.524) (layers "*.Cu" "*.Paste" "*.Mask") (drill 0.8) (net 2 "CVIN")))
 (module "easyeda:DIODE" (layer "F.Cu") (at 8.255 107.442 -90)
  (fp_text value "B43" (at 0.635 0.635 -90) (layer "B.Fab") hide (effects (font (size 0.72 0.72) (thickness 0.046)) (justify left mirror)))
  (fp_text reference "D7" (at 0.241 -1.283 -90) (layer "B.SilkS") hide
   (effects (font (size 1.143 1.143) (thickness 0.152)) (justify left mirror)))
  (pad 1 thru_hole circle (at 2.54 0 -90) (size 1.524 1.524) (layers "*.Cu" "*.Paste" "*.Mask") (drill 0.8) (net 2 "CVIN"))
  (pad 2 thru_hole circle (at -2.54 0 -90) (size 1.524 1.524) (layers "*.Cu" "*.Paste" "*.Mask") (drill 0.8) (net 11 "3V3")))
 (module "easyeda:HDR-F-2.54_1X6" (layer "F.Cu") (at 13.97 112.522)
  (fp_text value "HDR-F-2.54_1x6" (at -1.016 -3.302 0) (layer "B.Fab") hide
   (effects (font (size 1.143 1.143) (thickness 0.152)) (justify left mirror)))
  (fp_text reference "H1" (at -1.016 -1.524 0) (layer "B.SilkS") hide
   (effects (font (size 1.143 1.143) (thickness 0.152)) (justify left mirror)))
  (pad 6 thru_hole circle (at -7.62 0 0) (size 1.575 1.575) (layers "*.Cu" "*.Paste" "*.Mask") (drill 0.889) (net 14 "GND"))
  (pad 5 thru_hole circle (at -5.08 0 0) (size 1.575 1.575) (layers "*.Cu" "*.Paste" "*.Mask") (drill 0.889) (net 19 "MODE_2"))
  (pad 4 thru_hole circle (at -2.54 0 0) (size 1.575 1.575) (layers "*.Cu" "*.Paste" "*.Mask") (drill 0.889) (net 7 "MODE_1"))
  (pad 3 thru_hole circle (at 0 0 0) (size 1.575 1.575) (layers "*.Cu" "*.Paste" "*.Mask") (drill 0.889) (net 11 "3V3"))
  (pad 2 thru_hole circle (at 2.54 0 0) (size 1.575 1.575) (layers "*.Cu" "*.Paste" "*.Mask") (drill 0.889) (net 13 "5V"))
  (pad 1 thru_hole rect (at 5.08 0 0) (size 1.575 1.575) (layers "*.Cu" "*.Paste" "*.Mask") (drill 0.889) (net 2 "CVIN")))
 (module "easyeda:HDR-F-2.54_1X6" (layer "F.Cu") (at 17.145 166.497)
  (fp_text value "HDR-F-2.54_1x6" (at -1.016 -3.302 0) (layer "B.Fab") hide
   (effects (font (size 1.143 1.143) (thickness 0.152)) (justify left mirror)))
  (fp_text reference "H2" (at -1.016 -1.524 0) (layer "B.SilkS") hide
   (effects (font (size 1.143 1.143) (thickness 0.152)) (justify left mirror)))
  (pad 6 thru_hole circle (at -7.62 0 0) (size 1.575 1.575) (layers "*.Cu" "*.Paste" "*.Mask") (drill 0.889) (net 14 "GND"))
  (pad 5 thru_hole circle (at -5.08 0 0) (size 1.575 1.575) (layers "*.Cu" "*.Paste" "*.Mask") (drill 0.889) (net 4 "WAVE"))
  (pad 4 thru_hole circle (at -2.54 0 0) (size 1.575 1.575) (layers "*.Cu" "*.Paste" "*.Mask") (drill 0.889) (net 10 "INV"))
  (pad 3 thru_hole circle (at 0 0 0) (size 1.575 1.575) (layers "*.Cu" "*.Paste" "*.Mask") (drill 0.889) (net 16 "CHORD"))
  (pad 2 thru_hole circle (at 2.54 0 0) (size 1.575 1.575) (layers "*.Cu" "*.Paste" "*.Mask") (drill 0.889) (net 8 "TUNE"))
  (pad 1 thru_hole rect (at 5.08 0 0) (size 1.575 1.575) (layers "*.Cu" "*.Paste" "*.Mask") (drill 0.889) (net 18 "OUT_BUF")))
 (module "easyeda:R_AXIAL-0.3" (layer "F.Cu") (at 17.78 130.937)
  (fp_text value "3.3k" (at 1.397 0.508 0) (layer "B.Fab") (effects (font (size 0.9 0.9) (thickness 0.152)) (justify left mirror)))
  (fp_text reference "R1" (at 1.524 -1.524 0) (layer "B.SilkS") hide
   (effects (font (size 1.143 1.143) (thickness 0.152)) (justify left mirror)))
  (pad 1 thru_hole circle (at 3.81 0 0) (size 1.88 1.88) (layers "*.Cu" "*.Paste" "*.Mask") (drill 0.899) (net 2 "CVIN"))
  (pad 2 thru_hole circle (at -3.81 0 0) (size 1.88 1.88) (layers "*.Cu" "*.Paste" "*.Mask") (drill 0.899) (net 14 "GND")))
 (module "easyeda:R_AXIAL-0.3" (layer "F.Cu") (at 18.415 151.892)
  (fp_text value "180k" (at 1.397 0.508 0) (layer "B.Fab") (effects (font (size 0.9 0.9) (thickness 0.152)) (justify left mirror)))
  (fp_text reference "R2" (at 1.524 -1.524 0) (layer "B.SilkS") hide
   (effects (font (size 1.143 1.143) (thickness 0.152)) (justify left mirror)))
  (pad 1 thru_hole circle (at 3.81 0 0) (size 1.88 1.88) (layers "*.Cu" "*.Paste" "*.Mask") (drill 0.899) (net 16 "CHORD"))
  (pad 2 thru_hole circle (at -3.81 0 0) (size 1.88 1.88) (layers "*.Cu" "*.Paste" "*.Mask") (drill 0.899) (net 17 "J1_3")))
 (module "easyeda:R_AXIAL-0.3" (layer "F.Cu") (at 14.605 133.477)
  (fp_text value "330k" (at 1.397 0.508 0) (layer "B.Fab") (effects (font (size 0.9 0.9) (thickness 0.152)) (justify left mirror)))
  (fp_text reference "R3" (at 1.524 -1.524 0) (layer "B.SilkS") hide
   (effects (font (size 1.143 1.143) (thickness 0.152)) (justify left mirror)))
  (pad 1 thru_hole circle (at 3.81 0 0) (size 1.88 1.88) (layers "*.Cu" "*.Paste" "*.Mask") (drill 0.899) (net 16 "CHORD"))
  (pad 2 thru_hole circle (at -3.81 0 0) (size 1.88 1.88) (layers "*.Cu" "*.Paste" "*.Mask") (drill 0.899) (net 14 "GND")))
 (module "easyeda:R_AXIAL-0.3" (layer "F.Cu") (at 22.225 113.157 -90)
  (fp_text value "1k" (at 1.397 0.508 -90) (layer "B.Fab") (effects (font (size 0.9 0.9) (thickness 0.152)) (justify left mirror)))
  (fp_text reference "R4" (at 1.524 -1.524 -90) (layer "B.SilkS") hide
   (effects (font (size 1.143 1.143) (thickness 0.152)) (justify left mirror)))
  (pad 1 thru_hole circle (at 3.81 0 -90) (size 1.88 1.88) (layers "*.Cu" "*.Paste" "*.Mask") (drill 0.899) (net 8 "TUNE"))
  (pad 2 thru_hole circle (at -3.81 0 -90) (size 1.88 1.88) (layers "*.Cu" "*.Paste" "*.Mask") (drill 0.899) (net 12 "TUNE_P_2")))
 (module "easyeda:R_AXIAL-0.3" (layer "F.Cu") (at 13.335 149.987)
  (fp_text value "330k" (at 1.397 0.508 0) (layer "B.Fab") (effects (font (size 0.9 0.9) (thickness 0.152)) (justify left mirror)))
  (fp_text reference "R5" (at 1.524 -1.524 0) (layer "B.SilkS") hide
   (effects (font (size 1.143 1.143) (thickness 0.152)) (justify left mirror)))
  (pad 1 thru_hole circle (at 3.81 0 0) (size 1.88 1.88) (layers "*.Cu" "*.Paste" "*.Mask") (drill 0.899) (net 10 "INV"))
  (pad 2 thru_hole circle (at -3.81 0 0) (size 1.88 1.88) (layers "*.Cu" "*.Paste" "*.Mask") (drill 0.899) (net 14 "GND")))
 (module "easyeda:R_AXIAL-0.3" (layer "F.Cu") (at 18.796 184.023 180)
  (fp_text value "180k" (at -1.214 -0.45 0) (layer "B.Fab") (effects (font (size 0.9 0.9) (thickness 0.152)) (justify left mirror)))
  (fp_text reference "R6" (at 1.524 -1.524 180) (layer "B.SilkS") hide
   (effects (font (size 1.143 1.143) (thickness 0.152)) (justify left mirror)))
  (pad 1 thru_hole circle (at 3.81 0 180) (size 1.88 1.88) (layers "*.Cu" "*.Paste" "*.Mask") (drill 0.899) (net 10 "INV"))
  (pad 2 thru_hole circle (at -3.81 0 180) (size 1.88 1.88) (layers "*.Cu" "*.Paste" "*.Mask") (drill 0.899) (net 9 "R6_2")))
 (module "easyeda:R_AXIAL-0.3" (layer "F.Cu") (at 18.415 163.322)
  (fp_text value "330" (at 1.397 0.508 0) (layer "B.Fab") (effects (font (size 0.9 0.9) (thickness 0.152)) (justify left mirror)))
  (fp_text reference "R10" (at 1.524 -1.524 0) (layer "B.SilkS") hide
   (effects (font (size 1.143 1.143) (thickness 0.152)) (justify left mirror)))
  (pad 1 thru_hole circle (at 3.81 0 0) (size 1.88 1.88) (layers "*.Cu" "*.Paste" "*.Mask") (drill 0.899) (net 18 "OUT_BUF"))
  (pad 2 thru_hole circle (at -3.81 0 0) (size 1.88 1.88) (layers "*.Cu" "*.Paste" "*.Mask") (drill 0.899) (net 15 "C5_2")))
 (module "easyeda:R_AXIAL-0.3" (layer "F.Cu") (at 22.225 141.097 90)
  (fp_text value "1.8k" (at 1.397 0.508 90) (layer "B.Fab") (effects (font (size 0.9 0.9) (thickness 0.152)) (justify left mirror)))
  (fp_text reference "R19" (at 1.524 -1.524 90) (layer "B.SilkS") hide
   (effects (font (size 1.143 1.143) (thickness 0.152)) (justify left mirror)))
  (pad 1 thru_hole circle (at 3.81 0 90) (size 1.88 1.88) (layers "*.Cu" "*.Paste" "*.Mask") (drill 0.899) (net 2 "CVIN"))
  (pad 2 thru_hole circle (at -3.81 0 90) (size 1.88 1.88) (layers "*.Cu" "*.Paste" "*.Mask") (drill 0.899) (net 1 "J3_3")))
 (via (at 13.99 158.545) (size 0.7) (drill 0.55) (layers "F.Cu" "B.Cu") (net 1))
 (via (at 17.966 153.007) (size 0.7) (drill 0.55) (layers "F.Cu" "B.Cu") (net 1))
 (via (at 19.063 108.054) (size 0.7) (drill 0.55) (layers "F.Cu" "B.Cu") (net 2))
 (via (at 17.963 156.387) (size 0.7) (drill 0.55) (layers "F.Cu" "B.Cu") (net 4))
 (via (at 8.897 184.275) (size 0.7) (drill 0.55) (layers "F.Cu" "B.Cu") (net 15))
 (via (at 20.178 150.316) (size 0.7) (drill 0.55) (layers "F.Cu" "B.Cu") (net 16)))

